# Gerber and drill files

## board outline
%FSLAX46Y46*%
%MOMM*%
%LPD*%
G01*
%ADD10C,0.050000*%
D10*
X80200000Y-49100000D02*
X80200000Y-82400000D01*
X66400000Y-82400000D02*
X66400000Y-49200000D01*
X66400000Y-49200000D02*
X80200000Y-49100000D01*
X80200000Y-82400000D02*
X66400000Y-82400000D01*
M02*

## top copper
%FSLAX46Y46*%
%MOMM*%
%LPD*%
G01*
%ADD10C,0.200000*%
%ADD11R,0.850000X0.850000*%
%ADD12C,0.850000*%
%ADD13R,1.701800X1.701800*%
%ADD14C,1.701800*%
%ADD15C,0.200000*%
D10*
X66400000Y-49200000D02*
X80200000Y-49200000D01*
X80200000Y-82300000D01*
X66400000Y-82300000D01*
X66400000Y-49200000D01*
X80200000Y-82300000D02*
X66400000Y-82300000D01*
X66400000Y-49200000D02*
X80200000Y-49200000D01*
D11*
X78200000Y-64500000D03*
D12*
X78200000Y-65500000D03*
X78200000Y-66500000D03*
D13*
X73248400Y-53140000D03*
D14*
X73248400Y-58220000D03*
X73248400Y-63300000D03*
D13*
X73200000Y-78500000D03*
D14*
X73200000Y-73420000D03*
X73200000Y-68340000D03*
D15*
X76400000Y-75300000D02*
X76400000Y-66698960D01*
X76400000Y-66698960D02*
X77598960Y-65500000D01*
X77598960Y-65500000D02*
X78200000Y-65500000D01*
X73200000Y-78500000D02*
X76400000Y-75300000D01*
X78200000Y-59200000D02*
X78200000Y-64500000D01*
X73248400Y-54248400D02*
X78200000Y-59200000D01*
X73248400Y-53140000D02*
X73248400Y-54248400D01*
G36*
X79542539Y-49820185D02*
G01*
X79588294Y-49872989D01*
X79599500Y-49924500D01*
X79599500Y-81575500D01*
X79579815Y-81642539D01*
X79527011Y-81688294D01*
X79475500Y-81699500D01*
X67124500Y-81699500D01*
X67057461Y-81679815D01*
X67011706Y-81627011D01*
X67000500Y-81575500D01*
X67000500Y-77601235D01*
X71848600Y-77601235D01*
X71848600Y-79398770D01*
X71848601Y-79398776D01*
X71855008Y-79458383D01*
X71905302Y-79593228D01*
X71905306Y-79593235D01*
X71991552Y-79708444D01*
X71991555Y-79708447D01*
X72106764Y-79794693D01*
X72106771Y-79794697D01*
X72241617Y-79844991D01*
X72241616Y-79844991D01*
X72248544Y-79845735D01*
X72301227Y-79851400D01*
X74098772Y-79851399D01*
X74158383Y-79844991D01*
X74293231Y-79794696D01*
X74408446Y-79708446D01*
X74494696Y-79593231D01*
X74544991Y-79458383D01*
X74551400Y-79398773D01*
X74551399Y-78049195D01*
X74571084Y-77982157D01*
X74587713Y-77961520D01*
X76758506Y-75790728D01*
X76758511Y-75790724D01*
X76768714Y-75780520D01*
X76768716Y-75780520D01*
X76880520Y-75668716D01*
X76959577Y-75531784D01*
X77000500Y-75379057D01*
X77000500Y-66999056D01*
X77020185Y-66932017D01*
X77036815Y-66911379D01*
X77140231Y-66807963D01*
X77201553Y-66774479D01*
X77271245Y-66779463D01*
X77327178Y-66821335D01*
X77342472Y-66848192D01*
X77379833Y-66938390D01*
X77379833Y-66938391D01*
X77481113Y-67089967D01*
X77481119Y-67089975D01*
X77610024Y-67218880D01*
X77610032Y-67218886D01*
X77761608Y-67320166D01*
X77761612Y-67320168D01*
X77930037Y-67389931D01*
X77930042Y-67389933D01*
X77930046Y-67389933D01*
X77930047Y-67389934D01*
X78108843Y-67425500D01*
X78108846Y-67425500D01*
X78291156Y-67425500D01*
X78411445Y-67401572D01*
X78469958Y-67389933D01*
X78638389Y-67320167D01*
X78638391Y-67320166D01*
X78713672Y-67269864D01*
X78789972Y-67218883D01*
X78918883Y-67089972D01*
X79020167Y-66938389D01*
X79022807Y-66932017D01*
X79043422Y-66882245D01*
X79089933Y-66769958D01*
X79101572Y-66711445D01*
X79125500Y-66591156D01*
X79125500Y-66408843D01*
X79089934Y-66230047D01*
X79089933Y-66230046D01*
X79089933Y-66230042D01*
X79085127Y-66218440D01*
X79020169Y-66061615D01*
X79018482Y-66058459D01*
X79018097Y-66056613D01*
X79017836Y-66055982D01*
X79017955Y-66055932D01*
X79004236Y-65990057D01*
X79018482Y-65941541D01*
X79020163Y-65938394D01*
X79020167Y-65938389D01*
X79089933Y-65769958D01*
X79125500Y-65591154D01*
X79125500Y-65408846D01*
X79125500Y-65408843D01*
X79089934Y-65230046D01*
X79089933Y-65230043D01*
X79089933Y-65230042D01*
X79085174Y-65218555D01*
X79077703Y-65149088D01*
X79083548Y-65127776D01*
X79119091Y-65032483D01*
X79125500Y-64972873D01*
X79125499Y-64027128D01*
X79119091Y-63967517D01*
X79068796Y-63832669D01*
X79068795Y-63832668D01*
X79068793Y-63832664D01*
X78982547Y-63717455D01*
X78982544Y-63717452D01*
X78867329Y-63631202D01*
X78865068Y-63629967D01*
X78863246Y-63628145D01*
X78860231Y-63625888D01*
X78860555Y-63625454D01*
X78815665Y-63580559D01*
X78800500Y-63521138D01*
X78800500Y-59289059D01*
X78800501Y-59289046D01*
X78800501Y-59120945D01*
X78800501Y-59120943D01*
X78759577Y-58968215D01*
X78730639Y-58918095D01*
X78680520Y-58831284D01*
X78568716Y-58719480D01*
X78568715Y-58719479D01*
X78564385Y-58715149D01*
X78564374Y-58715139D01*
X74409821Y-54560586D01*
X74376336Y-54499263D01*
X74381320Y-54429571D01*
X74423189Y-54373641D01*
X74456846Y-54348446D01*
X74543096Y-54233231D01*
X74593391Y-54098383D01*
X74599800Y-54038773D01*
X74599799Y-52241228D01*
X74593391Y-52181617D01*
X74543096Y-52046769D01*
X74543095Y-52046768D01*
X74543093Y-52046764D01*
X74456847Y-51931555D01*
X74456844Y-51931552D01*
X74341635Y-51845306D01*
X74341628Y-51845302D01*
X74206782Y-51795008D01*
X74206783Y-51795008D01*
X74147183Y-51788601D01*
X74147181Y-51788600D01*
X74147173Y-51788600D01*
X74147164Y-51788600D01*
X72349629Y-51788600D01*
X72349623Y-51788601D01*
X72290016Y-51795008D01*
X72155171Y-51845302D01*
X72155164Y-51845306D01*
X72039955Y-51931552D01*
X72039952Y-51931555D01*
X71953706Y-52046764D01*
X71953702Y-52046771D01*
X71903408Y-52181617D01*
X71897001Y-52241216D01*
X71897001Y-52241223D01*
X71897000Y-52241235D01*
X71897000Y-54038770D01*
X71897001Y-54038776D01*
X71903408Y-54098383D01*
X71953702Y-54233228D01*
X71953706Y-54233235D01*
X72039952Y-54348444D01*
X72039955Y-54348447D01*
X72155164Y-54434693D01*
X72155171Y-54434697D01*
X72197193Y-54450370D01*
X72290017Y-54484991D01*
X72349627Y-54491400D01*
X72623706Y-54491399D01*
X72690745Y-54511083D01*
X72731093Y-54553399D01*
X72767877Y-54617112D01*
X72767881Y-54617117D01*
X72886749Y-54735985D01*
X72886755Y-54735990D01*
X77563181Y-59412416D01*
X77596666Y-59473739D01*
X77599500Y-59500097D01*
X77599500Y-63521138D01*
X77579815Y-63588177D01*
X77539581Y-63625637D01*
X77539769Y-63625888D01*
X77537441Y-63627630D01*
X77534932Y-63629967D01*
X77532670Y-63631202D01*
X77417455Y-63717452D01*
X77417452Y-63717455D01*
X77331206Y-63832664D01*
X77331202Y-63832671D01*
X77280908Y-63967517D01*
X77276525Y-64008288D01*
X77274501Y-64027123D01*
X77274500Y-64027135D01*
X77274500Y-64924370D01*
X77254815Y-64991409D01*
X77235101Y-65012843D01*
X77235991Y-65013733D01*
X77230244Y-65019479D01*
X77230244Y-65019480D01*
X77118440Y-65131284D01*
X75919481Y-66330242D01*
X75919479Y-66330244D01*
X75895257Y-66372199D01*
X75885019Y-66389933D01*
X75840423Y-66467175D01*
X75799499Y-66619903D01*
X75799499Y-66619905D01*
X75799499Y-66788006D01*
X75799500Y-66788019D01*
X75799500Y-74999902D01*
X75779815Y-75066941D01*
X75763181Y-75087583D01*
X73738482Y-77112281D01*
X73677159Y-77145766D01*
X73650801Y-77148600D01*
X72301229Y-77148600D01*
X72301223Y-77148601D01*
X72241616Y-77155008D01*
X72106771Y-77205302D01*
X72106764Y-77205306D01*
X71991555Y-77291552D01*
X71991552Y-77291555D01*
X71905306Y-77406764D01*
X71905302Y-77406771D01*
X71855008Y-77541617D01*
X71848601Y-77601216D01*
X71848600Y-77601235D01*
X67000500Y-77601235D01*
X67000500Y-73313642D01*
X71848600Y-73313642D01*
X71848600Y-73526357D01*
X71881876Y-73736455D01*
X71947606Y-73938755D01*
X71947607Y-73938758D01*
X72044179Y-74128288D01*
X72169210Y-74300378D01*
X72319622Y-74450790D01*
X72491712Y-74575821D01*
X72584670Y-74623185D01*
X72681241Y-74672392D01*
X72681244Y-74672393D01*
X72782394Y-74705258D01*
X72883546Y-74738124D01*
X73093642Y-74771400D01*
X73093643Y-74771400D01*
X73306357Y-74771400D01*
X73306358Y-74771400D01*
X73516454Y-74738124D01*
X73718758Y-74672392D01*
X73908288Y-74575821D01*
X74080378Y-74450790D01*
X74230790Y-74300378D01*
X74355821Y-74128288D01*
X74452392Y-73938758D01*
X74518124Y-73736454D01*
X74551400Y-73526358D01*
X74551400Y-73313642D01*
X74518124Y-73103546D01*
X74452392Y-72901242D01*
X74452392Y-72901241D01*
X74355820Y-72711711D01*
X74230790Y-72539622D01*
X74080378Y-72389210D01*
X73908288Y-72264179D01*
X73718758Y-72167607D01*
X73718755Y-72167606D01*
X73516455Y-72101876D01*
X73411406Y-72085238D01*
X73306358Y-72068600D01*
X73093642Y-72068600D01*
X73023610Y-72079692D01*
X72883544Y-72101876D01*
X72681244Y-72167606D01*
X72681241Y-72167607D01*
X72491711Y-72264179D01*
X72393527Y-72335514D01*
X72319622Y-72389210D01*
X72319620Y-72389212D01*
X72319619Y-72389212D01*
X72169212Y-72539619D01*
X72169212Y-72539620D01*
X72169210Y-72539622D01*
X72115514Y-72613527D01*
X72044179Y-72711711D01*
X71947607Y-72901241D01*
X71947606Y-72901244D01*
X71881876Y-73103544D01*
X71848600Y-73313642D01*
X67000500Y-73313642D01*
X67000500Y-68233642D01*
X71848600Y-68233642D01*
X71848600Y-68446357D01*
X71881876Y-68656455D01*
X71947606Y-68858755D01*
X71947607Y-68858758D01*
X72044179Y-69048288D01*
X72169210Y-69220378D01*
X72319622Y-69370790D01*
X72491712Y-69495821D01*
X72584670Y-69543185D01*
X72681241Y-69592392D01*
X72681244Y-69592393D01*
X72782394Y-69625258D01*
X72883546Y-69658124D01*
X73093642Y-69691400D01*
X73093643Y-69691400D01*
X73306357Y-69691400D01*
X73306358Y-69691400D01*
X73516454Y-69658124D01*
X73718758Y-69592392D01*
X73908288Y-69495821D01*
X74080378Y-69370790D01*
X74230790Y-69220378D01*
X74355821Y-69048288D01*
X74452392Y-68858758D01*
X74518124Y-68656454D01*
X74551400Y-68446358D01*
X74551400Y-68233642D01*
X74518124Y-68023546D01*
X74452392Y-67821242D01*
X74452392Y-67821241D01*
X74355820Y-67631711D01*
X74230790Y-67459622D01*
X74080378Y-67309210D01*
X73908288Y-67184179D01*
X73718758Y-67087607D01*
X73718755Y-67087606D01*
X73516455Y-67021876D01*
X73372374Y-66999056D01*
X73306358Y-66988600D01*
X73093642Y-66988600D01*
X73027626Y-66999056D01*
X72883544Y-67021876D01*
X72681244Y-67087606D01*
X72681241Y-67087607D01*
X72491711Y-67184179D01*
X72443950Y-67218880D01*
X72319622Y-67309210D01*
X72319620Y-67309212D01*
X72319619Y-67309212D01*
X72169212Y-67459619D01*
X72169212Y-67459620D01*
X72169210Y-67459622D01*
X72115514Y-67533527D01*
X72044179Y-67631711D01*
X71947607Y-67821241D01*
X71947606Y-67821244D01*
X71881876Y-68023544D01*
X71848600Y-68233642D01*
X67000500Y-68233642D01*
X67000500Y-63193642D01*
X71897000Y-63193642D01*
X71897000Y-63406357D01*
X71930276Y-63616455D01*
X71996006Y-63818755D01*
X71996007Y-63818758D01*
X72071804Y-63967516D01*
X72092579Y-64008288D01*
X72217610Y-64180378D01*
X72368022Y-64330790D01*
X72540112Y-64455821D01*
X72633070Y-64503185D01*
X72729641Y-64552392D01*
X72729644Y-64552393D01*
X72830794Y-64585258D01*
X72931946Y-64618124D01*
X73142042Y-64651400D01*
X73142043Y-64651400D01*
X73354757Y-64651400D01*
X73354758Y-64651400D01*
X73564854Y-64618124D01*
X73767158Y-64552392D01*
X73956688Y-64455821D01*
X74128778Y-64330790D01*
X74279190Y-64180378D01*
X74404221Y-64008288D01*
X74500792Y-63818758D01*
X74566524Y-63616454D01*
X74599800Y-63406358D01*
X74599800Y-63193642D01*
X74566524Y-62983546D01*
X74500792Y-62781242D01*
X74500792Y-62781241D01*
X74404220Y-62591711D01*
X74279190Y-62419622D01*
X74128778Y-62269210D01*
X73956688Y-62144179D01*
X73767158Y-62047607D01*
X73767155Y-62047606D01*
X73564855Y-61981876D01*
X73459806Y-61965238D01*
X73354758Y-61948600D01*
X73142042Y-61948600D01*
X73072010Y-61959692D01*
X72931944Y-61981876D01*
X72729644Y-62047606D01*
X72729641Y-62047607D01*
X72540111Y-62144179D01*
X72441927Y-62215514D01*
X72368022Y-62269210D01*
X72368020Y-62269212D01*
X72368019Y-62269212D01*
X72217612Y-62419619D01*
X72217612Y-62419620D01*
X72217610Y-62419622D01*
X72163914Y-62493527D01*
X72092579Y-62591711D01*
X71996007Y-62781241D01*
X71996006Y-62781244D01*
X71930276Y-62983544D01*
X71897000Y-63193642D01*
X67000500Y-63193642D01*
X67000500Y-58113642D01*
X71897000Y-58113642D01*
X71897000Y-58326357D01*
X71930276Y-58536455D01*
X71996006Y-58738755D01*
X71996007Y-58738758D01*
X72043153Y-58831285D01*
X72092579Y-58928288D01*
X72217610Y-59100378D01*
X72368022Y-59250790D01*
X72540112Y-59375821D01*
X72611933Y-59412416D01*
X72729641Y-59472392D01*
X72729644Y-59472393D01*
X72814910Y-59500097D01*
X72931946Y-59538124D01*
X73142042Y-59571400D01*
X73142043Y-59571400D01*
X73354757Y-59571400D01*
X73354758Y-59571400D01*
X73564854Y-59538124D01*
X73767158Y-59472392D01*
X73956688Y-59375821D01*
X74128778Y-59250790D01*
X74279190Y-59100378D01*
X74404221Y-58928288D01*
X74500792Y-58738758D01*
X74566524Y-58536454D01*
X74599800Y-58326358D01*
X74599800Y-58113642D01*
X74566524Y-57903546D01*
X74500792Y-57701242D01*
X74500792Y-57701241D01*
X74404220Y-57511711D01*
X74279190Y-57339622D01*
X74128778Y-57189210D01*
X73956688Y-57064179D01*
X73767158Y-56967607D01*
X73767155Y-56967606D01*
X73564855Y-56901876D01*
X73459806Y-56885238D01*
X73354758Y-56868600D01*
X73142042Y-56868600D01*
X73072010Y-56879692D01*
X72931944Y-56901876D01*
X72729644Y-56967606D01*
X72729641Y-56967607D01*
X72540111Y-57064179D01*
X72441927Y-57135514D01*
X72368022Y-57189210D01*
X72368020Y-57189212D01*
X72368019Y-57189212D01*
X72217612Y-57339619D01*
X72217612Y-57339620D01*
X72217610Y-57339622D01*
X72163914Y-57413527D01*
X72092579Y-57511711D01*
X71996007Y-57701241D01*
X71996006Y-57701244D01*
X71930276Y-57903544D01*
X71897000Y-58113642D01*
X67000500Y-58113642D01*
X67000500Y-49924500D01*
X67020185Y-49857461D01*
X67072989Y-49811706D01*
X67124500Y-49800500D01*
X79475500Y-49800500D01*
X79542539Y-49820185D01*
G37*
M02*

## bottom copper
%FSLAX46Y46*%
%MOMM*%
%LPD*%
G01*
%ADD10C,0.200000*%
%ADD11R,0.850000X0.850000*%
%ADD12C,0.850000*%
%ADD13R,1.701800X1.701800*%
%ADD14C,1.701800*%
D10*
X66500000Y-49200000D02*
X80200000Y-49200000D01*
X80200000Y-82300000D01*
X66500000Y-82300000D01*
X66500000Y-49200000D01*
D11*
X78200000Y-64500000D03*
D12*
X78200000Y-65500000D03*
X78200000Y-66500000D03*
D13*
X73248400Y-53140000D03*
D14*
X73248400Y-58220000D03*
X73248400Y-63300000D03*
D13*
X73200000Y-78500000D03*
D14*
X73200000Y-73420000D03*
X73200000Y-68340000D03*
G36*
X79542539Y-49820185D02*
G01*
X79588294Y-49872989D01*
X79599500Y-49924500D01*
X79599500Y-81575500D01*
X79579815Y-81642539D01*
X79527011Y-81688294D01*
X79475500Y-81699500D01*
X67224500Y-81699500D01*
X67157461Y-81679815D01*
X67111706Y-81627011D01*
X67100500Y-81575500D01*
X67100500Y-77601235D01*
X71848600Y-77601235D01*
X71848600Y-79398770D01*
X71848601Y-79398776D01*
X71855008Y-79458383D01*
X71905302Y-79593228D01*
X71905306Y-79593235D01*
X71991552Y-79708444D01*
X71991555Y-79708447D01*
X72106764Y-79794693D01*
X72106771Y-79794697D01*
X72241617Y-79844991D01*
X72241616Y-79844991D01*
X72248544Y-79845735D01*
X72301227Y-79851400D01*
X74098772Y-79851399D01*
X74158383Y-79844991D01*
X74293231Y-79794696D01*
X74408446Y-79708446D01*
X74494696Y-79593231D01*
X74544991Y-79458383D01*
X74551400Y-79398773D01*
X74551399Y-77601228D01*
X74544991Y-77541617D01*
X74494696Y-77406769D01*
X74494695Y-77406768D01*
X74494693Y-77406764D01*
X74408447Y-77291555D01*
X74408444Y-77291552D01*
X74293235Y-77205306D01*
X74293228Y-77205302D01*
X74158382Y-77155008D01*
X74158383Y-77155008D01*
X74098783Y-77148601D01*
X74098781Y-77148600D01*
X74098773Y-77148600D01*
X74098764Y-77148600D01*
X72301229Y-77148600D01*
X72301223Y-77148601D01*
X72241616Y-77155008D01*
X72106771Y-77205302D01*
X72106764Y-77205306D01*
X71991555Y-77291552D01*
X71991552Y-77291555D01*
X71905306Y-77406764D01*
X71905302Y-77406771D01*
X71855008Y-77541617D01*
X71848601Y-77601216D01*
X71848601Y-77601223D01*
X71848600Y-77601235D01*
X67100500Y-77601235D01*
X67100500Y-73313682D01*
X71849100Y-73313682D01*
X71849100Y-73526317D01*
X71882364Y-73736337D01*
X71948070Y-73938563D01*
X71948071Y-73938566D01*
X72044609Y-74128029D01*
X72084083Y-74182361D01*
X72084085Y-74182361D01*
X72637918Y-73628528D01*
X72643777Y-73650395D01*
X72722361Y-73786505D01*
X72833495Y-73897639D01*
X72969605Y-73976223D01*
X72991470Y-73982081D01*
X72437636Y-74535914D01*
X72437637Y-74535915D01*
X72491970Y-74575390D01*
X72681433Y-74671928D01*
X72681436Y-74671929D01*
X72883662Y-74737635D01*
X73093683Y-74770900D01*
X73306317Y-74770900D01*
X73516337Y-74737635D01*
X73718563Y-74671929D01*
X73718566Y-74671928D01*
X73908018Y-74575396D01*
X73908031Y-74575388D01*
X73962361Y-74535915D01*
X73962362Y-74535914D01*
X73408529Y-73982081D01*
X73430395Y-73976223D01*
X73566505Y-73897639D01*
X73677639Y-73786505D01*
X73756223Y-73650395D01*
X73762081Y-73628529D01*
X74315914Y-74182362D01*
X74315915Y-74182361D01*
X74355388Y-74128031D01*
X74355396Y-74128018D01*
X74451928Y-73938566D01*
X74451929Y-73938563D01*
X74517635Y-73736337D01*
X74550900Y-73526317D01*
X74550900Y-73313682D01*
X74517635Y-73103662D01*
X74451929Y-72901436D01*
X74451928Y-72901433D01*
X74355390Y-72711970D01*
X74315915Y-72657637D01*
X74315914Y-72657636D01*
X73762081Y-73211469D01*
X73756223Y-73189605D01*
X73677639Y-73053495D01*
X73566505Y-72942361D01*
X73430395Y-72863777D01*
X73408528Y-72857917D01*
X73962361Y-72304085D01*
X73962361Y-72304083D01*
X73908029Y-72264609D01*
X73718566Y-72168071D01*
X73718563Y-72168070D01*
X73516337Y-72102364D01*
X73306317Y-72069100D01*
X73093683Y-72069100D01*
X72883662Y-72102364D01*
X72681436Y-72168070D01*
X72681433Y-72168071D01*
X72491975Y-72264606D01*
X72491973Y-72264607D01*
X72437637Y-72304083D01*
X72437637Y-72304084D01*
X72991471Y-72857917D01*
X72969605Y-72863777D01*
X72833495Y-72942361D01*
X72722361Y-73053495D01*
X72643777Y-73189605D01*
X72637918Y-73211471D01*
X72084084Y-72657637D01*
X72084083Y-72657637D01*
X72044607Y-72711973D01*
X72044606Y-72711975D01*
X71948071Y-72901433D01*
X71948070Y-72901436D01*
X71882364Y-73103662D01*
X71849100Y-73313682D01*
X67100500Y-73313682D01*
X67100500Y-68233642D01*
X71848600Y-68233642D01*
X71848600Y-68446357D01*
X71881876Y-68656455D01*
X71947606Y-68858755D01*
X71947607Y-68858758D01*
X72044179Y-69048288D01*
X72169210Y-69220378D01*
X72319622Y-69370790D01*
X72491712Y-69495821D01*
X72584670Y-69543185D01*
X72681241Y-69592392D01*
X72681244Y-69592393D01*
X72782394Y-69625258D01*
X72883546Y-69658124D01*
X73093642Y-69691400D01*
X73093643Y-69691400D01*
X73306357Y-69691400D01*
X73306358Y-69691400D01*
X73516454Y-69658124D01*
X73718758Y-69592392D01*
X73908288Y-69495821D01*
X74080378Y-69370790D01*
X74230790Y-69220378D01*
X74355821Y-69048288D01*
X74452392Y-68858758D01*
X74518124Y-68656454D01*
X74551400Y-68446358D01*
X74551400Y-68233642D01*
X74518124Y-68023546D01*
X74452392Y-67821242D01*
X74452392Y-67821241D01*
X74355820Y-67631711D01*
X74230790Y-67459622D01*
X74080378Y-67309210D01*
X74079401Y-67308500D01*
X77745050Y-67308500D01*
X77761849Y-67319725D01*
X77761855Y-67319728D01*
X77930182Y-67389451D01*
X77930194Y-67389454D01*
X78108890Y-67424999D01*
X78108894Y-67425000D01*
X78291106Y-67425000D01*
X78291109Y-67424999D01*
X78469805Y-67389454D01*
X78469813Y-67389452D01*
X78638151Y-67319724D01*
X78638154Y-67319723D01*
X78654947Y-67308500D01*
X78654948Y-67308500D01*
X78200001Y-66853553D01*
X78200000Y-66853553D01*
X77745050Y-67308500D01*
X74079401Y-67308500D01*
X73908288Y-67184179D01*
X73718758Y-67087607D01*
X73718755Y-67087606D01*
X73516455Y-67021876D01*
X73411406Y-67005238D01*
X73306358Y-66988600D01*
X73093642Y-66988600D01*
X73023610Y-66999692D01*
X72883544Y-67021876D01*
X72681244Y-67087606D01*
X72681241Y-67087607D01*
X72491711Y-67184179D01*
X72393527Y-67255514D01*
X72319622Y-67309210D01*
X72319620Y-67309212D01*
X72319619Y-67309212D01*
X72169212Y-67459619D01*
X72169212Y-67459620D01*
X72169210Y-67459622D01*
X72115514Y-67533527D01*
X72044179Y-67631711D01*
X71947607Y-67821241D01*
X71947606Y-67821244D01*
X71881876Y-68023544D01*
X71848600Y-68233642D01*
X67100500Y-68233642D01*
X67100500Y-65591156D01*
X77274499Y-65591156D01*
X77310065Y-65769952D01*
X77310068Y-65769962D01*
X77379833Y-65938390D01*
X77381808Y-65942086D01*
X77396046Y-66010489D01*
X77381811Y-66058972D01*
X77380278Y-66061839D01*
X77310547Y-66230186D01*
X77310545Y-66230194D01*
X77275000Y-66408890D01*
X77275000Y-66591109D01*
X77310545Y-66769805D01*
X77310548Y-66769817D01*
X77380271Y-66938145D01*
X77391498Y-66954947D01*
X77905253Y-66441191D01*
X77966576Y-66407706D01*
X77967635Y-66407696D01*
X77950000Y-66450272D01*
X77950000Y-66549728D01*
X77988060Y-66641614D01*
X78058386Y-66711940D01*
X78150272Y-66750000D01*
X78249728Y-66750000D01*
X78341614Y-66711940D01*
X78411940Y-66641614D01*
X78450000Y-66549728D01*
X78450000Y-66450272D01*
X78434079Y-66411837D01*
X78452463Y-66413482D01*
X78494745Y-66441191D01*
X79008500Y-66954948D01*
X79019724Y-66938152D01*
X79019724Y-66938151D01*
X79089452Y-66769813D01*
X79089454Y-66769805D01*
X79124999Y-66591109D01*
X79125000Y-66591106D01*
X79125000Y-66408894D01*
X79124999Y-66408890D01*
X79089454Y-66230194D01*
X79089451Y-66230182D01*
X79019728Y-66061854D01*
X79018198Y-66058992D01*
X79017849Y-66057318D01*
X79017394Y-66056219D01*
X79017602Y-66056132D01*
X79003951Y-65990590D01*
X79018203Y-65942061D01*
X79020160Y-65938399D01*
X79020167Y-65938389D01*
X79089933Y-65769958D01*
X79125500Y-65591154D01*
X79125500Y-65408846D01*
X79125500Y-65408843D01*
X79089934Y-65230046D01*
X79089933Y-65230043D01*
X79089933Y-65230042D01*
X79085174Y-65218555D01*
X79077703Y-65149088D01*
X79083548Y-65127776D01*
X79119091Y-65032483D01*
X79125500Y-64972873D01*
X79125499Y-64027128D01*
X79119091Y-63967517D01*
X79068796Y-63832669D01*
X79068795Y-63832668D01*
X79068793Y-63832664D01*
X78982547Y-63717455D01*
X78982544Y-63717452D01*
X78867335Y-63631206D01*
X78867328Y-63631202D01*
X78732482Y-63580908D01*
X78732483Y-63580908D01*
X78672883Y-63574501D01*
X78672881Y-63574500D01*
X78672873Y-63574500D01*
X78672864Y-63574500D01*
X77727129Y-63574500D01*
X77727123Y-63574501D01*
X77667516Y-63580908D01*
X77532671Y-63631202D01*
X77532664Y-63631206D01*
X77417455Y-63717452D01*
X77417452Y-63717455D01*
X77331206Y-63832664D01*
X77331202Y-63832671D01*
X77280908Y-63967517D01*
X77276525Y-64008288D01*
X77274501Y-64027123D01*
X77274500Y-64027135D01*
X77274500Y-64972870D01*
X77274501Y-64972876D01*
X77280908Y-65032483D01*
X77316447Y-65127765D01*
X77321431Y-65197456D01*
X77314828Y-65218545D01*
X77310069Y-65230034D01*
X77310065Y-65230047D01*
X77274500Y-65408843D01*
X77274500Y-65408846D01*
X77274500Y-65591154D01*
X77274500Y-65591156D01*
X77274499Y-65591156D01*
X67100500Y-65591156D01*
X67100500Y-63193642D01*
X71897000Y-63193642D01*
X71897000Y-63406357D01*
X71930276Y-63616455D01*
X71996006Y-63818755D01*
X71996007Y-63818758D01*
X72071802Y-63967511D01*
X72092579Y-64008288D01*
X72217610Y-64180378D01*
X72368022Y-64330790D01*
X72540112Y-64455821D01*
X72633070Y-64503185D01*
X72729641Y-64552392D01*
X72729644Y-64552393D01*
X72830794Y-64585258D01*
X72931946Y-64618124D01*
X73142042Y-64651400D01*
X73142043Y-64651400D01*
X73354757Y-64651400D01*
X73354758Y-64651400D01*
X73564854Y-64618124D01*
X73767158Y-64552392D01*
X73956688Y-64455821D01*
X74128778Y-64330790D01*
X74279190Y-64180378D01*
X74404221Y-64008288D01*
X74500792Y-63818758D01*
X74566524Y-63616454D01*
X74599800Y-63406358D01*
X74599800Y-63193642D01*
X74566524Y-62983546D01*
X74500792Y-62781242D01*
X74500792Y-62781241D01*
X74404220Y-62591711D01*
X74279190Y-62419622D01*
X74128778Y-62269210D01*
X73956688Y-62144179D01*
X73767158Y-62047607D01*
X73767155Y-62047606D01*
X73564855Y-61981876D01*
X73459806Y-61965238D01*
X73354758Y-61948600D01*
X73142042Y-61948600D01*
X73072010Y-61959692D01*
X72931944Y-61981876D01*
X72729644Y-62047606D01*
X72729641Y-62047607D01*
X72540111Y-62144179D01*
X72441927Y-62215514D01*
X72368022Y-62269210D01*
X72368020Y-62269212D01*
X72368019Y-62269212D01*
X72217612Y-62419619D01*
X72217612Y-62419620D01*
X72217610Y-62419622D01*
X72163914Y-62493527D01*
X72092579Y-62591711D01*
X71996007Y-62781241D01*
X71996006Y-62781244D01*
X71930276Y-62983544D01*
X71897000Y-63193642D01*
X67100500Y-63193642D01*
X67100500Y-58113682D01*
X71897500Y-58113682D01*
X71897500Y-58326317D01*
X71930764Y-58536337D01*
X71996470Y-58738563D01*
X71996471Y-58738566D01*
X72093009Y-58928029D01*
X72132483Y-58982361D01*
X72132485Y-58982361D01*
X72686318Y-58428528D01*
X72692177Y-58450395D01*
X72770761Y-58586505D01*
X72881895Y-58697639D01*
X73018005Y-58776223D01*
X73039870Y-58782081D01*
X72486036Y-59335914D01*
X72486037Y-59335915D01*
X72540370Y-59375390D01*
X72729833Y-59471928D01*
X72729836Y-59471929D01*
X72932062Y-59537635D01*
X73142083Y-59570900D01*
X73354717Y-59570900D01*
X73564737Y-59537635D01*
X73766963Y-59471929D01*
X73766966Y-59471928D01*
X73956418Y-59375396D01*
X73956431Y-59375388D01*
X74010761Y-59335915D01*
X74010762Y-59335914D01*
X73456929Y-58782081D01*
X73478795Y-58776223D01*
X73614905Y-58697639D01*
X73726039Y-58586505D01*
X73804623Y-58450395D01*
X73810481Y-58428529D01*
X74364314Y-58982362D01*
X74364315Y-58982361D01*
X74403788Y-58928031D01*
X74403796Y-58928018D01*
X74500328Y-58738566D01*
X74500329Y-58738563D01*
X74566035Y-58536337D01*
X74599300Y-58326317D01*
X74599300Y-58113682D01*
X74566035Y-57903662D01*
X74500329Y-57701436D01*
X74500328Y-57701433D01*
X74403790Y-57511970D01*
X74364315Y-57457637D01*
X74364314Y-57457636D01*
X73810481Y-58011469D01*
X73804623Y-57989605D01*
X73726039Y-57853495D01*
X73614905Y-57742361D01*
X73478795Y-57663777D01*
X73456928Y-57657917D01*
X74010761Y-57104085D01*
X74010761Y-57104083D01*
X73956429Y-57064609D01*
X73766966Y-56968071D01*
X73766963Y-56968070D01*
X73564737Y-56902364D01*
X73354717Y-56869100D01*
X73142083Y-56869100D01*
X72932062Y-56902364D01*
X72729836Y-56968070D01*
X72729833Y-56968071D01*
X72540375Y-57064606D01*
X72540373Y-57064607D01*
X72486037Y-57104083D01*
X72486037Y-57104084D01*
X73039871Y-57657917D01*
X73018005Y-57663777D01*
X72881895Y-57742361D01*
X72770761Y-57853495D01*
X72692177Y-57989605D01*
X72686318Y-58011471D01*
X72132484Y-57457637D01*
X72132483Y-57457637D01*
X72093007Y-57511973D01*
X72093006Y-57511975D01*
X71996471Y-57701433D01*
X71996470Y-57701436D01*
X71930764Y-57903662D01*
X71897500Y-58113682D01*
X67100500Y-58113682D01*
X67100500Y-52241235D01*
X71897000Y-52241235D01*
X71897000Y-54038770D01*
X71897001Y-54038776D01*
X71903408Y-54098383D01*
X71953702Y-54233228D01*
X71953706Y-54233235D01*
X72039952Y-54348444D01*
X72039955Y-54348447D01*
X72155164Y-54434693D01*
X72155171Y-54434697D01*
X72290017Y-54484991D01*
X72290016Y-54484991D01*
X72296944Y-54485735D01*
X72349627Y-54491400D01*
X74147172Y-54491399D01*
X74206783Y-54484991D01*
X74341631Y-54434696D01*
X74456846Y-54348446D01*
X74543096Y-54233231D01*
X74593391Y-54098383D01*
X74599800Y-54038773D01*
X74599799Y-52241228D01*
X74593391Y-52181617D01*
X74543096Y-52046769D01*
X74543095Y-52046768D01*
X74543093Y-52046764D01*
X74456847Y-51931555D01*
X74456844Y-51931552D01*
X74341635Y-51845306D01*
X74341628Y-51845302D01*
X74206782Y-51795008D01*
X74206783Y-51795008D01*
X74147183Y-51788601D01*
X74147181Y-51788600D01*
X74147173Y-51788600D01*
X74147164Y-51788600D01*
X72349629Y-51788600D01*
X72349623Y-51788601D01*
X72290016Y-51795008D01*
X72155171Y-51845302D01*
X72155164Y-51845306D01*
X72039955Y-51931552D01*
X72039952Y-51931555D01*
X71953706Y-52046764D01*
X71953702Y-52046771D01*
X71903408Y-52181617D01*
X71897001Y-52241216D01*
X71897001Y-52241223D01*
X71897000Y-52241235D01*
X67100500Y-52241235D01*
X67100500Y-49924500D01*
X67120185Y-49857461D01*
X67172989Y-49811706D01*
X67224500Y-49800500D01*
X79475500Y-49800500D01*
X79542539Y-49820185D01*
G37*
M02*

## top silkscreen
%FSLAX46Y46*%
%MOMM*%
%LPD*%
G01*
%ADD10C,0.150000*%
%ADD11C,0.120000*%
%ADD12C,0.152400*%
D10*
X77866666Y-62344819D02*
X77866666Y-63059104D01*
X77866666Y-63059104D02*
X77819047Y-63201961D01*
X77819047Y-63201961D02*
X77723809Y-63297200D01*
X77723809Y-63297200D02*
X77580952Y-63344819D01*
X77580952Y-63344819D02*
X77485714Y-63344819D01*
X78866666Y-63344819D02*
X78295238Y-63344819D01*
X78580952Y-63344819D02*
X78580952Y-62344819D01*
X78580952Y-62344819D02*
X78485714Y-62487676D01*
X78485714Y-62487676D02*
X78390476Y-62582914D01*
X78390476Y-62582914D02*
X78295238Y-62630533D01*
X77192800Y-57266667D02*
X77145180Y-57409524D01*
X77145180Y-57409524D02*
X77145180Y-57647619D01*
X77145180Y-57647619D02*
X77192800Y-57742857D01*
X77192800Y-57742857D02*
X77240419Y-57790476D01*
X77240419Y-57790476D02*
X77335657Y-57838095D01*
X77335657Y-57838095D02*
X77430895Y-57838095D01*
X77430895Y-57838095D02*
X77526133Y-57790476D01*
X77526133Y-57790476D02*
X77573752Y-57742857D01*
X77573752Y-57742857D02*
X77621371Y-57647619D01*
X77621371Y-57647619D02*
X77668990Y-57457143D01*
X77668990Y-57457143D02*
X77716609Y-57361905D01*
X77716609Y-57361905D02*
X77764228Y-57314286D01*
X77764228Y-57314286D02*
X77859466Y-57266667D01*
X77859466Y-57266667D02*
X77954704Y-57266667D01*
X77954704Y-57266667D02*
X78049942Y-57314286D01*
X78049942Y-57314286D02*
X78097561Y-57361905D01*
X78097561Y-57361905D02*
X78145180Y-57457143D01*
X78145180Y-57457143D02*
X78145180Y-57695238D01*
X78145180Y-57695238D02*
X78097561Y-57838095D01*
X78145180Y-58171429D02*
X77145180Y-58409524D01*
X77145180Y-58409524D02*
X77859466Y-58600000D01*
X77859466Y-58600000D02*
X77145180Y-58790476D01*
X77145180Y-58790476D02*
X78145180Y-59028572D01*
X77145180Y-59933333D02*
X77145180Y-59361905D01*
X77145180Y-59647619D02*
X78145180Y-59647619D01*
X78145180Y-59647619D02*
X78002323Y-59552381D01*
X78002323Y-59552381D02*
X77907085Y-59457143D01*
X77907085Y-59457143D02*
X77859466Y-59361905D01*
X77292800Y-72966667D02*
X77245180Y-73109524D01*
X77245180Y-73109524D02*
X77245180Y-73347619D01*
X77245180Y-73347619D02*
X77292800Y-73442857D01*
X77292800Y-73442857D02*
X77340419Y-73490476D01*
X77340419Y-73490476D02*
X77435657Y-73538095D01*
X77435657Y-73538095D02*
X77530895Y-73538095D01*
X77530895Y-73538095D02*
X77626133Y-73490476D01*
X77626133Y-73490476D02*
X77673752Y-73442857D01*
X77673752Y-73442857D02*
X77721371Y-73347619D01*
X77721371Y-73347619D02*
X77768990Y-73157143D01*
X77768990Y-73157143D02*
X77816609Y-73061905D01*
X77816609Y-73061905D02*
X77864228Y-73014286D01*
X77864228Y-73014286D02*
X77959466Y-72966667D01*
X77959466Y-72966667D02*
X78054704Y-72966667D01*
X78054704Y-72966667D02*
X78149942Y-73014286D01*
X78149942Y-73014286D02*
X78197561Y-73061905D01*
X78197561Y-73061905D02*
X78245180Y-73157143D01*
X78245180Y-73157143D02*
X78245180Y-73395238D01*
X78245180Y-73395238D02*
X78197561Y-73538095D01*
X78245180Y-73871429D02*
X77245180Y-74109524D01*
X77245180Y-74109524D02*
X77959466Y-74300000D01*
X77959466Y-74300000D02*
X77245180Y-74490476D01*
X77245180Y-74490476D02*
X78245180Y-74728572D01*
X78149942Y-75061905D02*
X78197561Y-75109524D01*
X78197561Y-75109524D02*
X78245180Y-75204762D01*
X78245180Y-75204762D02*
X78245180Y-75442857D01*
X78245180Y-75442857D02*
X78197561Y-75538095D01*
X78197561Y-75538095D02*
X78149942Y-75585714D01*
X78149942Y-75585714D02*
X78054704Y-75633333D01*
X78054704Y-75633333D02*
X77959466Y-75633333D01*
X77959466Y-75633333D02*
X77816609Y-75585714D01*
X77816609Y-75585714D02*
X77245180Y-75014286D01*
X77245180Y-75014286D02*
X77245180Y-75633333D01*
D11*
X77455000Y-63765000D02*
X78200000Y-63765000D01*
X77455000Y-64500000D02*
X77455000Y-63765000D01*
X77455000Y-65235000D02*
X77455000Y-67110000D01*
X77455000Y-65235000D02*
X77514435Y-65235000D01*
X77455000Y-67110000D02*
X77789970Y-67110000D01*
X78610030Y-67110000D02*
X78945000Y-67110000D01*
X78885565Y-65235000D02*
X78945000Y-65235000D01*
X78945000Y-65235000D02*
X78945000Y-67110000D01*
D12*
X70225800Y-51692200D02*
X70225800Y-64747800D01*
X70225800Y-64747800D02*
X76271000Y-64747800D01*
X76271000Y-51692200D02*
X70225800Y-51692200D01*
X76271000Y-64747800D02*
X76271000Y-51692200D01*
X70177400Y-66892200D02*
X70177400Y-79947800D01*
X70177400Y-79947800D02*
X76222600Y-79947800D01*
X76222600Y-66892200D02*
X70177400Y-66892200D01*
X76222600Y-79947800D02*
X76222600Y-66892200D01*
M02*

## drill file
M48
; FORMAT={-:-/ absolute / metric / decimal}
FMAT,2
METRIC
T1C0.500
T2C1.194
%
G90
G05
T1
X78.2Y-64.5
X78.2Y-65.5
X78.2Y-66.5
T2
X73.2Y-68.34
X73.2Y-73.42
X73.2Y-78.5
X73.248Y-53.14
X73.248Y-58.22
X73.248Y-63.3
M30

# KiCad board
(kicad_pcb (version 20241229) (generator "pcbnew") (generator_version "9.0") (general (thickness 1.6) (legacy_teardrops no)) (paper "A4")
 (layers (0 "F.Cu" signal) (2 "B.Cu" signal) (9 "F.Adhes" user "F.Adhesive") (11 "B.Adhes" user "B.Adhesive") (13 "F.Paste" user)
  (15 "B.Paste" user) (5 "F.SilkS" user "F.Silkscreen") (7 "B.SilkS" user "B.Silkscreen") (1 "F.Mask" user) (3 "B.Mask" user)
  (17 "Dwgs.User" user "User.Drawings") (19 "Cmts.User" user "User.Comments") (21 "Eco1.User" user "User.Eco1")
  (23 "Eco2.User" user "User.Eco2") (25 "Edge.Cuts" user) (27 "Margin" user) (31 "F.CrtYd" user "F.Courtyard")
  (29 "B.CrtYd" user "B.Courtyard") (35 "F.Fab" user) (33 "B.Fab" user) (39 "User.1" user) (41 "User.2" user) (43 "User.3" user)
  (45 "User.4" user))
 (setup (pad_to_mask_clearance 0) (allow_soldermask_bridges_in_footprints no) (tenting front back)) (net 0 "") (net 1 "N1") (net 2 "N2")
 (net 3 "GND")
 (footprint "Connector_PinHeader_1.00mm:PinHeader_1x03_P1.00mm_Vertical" (layer "F.Cu") (at 78.2 64.5)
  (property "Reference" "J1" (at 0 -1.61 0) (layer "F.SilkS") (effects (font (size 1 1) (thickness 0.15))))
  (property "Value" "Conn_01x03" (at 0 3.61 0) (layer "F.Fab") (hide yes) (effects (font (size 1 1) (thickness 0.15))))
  (fp_line (start -0.745 -0.735) (end 0 -0.735) (stroke (width 0.12) (type solid)) (layer "F.SilkS"))
  (fp_line (start -0.745 0) (end -0.745 -0.735) (stroke (width 0.12) (type solid)) (layer "F.SilkS"))
  (fp_line (start -0.745 0.735) (end -0.745 2.61) (stroke (width 0.12) (type solid)) (layer "F.SilkS"))
  (fp_line (start -0.745 0.735) (end -0.685565 0.735) (stroke (width 0.12) (type solid)) (layer "F.SilkS"))
  (fp_line (start -0.745 2.61) (end -0.41003 2.61) (stroke (width 0.12) (type solid)) (layer "F.SilkS"))
  (fp_line (start 0.41003 2.61) (end 0.745 2.61) (stroke (width 0.12) (type solid)) (layer "F.SilkS"))
  (fp_line (start 0.685565 0.735) (end 0.745 0.735) (stroke (width 0.12) (type solid)) (layer "F.SilkS"))
  (fp_line (start 0.745 0.735) (end 0.745 2.61) (stroke (width 0.12) (type solid)) (layer "F.SilkS"))
  (pad "1" thru_hole rect (at 0 0) (size 0.85 0.85) (drill 0.5) (layers "*.Cu" "*.Mask") (remove_unused_layers no) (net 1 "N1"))
  (pad "2" thru_hole circle (at 0 1) (size 0.85 0.85) (drill 0.5) (layers "*.Cu" "*.Mask") (remove_unused_layers no) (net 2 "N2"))
  (pad "3" thru_hole circle (at 0 2) (size 0.85 0.85) (drill 0.5) (layers "*.Cu" "*.Mask") (remove_unused_layers no) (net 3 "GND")))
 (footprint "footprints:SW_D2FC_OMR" (layer "F.Cu") (at 73.2484 53.14)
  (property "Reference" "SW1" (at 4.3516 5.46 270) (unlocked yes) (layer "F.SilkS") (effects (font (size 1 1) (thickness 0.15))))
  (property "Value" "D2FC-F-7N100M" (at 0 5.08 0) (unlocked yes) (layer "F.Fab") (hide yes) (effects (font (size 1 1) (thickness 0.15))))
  (fp_line (start -3.0226 -1.4478) (end -3.0226 11.6078) (stroke (width 0.1524) (type solid)) (layer "F.SilkS"))
  (fp_line (start -3.0226 11.6078) (end 3.0226 11.6078) (stroke (width 0.1524) (type solid)) (layer "F.SilkS"))
  (fp_line (start 3.0226 -1.4478) (end -3.0226 -1.4478) (stroke (width 0.1524) (type solid)) (layer "F.SilkS"))
  (fp_line (start 3.0226 11.6078) (end 3.0226 -1.4478) (stroke (width 0.1524) (type solid)) (layer "F.SilkS"))
  (pad "1" thru_hole rect (at 0 0) (size 1.7018 1.7018) (drill 1.1938) (layers "*.Cu" "*.Mask") (remove_unused_layers no) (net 1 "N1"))
  (pad "2" thru_hole circle (at 0 5.08) (size 1.7018 1.7018) (drill 1.1938) (layers "*.Cu" "*.Mask") (remove_unused_layers no) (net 3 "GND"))
  (pad "3" thru_hole circle (at 0 10.16) (size 1.7018 1.7018) (drill 1.1938) (layers "*.Cu" "*.Mask") (remove_unused_layers no)))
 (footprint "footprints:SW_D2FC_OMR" (layer "F.Cu") (at 73.2 78.5 180)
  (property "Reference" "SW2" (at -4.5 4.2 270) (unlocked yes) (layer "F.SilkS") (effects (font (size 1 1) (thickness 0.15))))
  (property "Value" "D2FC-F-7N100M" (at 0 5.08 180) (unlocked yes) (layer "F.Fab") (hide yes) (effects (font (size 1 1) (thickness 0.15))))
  (fp_line (start 3.0226 11.6078) (end 3.0226 -1.4478) (stroke (width 0.1524) (type solid)) (layer "F.SilkS"))
  (fp_line (start 3.0226 -1.4478) (end -3.0226 -1.4478) (stroke (width 0.1524) (type solid)) (layer "F.SilkS"))
  (fp_line (start -3.0226 11.6078) (end 3.0226 11.6078) (stroke (width 0.1524) (type solid)) (layer "F.SilkS"))
  (fp_line (start -3.0226 -1.4478) (end -3.0226 11.6078) (stroke (width 0.1524) (type solid)) (layer "F.SilkS"))
  (pad "1" thru_hole rect (at 0 0 180) (size 1.7018 1.7018) (drill 1.1938) (layers "*.Cu" "*.Mask") (remove_unused_layers no) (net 2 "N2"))
  (pad "2" thru_hole circle (at 0 5.08 180) (size 1.7018 1.7018) (drill 1.1938) (layers "*.Cu" "*.Mask") (remove_unused_layers no)
   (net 3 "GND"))
  (pad "3" thru_hole circle (at 0 10.16 180) (size 1.7018 1.7018) (drill 1.1938) (layers "*.Cu" "*.Mask") (remove_unused_layers no)))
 (gr_rect (start 66.4 49.2) (end 80.2 82.3) (stroke (width 0.2) (type default)) (fill no) (layer "F.Cu"))
 (gr_line (start 80.2 82.3) (end 66.4 82.3) (stroke (width 0.2) (type default)) (layer "F.Cu"))
 (gr_line (start 66.4 49.2) (end 80.2 49.2) (stroke (width 0.2) (type default)) (layer "F.Cu"))
 (gr_rect (start 66.5 49.2) (end 80.2 82.3) (stroke (width 0.2) (type default)) (fill no) (layer "B.Cu"))
 (gr_line (start 80.2 49.1) (end 80.2 82.4) (stroke (width 0.05) (type default)) (layer "Edge.Cuts"))
 (gr_line (start 66.4 82.4) (end 66.4 49.2) (stroke (width 0.05) (type default)) (layer "Edge.Cuts"))
 (gr_line (start 66.4 49.2) (end 80.2 49.1) (stroke (width 0.05) (type default)) (layer "Edge.Cuts"))
 (gr_line (start 80.2 82.4) (end 66.4 82.4) (stroke (width 0.05) (type default)) (layer "Edge.Cuts"))
 (segment (start 76.4 75.3) (end 76.4 66.69896) (width 0.2) (layer "F.Cu") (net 2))
 (segment (start 76.4 66.69896) (end 77.59896 65.5) (width 0.2) (layer "F.Cu") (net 2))
 (segment (start 77.59896 65.5) (end 78.2 65.5) (width 0.2) (layer "F.Cu") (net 2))
 (segment (start 73.2 78.5) (end 76.4 75.3) (width 0.2) (layer "F.Cu") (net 2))
 (segment (start 78.2 59.2) (end 78.2 64.5) (width 0.2) (layer "F.Cu") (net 1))
 (segment (start 73.2484 54.2484) (end 78.2 59.2) (width 0.2) (layer "F.Cu") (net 1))
 (segment (start 73.2484 53.14) (end 73.2484 54.2484) (width 0.2) (layer "F.Cu") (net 1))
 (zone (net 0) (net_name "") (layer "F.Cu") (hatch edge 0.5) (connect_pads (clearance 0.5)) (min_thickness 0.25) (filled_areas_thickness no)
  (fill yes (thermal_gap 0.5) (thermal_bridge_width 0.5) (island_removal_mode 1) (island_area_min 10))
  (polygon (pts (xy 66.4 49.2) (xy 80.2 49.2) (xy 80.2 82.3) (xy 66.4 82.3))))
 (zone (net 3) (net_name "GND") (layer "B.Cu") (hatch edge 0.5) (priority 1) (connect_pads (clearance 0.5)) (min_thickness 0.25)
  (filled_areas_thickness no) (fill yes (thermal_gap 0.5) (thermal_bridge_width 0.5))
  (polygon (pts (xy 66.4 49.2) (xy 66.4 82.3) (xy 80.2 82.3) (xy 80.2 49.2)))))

